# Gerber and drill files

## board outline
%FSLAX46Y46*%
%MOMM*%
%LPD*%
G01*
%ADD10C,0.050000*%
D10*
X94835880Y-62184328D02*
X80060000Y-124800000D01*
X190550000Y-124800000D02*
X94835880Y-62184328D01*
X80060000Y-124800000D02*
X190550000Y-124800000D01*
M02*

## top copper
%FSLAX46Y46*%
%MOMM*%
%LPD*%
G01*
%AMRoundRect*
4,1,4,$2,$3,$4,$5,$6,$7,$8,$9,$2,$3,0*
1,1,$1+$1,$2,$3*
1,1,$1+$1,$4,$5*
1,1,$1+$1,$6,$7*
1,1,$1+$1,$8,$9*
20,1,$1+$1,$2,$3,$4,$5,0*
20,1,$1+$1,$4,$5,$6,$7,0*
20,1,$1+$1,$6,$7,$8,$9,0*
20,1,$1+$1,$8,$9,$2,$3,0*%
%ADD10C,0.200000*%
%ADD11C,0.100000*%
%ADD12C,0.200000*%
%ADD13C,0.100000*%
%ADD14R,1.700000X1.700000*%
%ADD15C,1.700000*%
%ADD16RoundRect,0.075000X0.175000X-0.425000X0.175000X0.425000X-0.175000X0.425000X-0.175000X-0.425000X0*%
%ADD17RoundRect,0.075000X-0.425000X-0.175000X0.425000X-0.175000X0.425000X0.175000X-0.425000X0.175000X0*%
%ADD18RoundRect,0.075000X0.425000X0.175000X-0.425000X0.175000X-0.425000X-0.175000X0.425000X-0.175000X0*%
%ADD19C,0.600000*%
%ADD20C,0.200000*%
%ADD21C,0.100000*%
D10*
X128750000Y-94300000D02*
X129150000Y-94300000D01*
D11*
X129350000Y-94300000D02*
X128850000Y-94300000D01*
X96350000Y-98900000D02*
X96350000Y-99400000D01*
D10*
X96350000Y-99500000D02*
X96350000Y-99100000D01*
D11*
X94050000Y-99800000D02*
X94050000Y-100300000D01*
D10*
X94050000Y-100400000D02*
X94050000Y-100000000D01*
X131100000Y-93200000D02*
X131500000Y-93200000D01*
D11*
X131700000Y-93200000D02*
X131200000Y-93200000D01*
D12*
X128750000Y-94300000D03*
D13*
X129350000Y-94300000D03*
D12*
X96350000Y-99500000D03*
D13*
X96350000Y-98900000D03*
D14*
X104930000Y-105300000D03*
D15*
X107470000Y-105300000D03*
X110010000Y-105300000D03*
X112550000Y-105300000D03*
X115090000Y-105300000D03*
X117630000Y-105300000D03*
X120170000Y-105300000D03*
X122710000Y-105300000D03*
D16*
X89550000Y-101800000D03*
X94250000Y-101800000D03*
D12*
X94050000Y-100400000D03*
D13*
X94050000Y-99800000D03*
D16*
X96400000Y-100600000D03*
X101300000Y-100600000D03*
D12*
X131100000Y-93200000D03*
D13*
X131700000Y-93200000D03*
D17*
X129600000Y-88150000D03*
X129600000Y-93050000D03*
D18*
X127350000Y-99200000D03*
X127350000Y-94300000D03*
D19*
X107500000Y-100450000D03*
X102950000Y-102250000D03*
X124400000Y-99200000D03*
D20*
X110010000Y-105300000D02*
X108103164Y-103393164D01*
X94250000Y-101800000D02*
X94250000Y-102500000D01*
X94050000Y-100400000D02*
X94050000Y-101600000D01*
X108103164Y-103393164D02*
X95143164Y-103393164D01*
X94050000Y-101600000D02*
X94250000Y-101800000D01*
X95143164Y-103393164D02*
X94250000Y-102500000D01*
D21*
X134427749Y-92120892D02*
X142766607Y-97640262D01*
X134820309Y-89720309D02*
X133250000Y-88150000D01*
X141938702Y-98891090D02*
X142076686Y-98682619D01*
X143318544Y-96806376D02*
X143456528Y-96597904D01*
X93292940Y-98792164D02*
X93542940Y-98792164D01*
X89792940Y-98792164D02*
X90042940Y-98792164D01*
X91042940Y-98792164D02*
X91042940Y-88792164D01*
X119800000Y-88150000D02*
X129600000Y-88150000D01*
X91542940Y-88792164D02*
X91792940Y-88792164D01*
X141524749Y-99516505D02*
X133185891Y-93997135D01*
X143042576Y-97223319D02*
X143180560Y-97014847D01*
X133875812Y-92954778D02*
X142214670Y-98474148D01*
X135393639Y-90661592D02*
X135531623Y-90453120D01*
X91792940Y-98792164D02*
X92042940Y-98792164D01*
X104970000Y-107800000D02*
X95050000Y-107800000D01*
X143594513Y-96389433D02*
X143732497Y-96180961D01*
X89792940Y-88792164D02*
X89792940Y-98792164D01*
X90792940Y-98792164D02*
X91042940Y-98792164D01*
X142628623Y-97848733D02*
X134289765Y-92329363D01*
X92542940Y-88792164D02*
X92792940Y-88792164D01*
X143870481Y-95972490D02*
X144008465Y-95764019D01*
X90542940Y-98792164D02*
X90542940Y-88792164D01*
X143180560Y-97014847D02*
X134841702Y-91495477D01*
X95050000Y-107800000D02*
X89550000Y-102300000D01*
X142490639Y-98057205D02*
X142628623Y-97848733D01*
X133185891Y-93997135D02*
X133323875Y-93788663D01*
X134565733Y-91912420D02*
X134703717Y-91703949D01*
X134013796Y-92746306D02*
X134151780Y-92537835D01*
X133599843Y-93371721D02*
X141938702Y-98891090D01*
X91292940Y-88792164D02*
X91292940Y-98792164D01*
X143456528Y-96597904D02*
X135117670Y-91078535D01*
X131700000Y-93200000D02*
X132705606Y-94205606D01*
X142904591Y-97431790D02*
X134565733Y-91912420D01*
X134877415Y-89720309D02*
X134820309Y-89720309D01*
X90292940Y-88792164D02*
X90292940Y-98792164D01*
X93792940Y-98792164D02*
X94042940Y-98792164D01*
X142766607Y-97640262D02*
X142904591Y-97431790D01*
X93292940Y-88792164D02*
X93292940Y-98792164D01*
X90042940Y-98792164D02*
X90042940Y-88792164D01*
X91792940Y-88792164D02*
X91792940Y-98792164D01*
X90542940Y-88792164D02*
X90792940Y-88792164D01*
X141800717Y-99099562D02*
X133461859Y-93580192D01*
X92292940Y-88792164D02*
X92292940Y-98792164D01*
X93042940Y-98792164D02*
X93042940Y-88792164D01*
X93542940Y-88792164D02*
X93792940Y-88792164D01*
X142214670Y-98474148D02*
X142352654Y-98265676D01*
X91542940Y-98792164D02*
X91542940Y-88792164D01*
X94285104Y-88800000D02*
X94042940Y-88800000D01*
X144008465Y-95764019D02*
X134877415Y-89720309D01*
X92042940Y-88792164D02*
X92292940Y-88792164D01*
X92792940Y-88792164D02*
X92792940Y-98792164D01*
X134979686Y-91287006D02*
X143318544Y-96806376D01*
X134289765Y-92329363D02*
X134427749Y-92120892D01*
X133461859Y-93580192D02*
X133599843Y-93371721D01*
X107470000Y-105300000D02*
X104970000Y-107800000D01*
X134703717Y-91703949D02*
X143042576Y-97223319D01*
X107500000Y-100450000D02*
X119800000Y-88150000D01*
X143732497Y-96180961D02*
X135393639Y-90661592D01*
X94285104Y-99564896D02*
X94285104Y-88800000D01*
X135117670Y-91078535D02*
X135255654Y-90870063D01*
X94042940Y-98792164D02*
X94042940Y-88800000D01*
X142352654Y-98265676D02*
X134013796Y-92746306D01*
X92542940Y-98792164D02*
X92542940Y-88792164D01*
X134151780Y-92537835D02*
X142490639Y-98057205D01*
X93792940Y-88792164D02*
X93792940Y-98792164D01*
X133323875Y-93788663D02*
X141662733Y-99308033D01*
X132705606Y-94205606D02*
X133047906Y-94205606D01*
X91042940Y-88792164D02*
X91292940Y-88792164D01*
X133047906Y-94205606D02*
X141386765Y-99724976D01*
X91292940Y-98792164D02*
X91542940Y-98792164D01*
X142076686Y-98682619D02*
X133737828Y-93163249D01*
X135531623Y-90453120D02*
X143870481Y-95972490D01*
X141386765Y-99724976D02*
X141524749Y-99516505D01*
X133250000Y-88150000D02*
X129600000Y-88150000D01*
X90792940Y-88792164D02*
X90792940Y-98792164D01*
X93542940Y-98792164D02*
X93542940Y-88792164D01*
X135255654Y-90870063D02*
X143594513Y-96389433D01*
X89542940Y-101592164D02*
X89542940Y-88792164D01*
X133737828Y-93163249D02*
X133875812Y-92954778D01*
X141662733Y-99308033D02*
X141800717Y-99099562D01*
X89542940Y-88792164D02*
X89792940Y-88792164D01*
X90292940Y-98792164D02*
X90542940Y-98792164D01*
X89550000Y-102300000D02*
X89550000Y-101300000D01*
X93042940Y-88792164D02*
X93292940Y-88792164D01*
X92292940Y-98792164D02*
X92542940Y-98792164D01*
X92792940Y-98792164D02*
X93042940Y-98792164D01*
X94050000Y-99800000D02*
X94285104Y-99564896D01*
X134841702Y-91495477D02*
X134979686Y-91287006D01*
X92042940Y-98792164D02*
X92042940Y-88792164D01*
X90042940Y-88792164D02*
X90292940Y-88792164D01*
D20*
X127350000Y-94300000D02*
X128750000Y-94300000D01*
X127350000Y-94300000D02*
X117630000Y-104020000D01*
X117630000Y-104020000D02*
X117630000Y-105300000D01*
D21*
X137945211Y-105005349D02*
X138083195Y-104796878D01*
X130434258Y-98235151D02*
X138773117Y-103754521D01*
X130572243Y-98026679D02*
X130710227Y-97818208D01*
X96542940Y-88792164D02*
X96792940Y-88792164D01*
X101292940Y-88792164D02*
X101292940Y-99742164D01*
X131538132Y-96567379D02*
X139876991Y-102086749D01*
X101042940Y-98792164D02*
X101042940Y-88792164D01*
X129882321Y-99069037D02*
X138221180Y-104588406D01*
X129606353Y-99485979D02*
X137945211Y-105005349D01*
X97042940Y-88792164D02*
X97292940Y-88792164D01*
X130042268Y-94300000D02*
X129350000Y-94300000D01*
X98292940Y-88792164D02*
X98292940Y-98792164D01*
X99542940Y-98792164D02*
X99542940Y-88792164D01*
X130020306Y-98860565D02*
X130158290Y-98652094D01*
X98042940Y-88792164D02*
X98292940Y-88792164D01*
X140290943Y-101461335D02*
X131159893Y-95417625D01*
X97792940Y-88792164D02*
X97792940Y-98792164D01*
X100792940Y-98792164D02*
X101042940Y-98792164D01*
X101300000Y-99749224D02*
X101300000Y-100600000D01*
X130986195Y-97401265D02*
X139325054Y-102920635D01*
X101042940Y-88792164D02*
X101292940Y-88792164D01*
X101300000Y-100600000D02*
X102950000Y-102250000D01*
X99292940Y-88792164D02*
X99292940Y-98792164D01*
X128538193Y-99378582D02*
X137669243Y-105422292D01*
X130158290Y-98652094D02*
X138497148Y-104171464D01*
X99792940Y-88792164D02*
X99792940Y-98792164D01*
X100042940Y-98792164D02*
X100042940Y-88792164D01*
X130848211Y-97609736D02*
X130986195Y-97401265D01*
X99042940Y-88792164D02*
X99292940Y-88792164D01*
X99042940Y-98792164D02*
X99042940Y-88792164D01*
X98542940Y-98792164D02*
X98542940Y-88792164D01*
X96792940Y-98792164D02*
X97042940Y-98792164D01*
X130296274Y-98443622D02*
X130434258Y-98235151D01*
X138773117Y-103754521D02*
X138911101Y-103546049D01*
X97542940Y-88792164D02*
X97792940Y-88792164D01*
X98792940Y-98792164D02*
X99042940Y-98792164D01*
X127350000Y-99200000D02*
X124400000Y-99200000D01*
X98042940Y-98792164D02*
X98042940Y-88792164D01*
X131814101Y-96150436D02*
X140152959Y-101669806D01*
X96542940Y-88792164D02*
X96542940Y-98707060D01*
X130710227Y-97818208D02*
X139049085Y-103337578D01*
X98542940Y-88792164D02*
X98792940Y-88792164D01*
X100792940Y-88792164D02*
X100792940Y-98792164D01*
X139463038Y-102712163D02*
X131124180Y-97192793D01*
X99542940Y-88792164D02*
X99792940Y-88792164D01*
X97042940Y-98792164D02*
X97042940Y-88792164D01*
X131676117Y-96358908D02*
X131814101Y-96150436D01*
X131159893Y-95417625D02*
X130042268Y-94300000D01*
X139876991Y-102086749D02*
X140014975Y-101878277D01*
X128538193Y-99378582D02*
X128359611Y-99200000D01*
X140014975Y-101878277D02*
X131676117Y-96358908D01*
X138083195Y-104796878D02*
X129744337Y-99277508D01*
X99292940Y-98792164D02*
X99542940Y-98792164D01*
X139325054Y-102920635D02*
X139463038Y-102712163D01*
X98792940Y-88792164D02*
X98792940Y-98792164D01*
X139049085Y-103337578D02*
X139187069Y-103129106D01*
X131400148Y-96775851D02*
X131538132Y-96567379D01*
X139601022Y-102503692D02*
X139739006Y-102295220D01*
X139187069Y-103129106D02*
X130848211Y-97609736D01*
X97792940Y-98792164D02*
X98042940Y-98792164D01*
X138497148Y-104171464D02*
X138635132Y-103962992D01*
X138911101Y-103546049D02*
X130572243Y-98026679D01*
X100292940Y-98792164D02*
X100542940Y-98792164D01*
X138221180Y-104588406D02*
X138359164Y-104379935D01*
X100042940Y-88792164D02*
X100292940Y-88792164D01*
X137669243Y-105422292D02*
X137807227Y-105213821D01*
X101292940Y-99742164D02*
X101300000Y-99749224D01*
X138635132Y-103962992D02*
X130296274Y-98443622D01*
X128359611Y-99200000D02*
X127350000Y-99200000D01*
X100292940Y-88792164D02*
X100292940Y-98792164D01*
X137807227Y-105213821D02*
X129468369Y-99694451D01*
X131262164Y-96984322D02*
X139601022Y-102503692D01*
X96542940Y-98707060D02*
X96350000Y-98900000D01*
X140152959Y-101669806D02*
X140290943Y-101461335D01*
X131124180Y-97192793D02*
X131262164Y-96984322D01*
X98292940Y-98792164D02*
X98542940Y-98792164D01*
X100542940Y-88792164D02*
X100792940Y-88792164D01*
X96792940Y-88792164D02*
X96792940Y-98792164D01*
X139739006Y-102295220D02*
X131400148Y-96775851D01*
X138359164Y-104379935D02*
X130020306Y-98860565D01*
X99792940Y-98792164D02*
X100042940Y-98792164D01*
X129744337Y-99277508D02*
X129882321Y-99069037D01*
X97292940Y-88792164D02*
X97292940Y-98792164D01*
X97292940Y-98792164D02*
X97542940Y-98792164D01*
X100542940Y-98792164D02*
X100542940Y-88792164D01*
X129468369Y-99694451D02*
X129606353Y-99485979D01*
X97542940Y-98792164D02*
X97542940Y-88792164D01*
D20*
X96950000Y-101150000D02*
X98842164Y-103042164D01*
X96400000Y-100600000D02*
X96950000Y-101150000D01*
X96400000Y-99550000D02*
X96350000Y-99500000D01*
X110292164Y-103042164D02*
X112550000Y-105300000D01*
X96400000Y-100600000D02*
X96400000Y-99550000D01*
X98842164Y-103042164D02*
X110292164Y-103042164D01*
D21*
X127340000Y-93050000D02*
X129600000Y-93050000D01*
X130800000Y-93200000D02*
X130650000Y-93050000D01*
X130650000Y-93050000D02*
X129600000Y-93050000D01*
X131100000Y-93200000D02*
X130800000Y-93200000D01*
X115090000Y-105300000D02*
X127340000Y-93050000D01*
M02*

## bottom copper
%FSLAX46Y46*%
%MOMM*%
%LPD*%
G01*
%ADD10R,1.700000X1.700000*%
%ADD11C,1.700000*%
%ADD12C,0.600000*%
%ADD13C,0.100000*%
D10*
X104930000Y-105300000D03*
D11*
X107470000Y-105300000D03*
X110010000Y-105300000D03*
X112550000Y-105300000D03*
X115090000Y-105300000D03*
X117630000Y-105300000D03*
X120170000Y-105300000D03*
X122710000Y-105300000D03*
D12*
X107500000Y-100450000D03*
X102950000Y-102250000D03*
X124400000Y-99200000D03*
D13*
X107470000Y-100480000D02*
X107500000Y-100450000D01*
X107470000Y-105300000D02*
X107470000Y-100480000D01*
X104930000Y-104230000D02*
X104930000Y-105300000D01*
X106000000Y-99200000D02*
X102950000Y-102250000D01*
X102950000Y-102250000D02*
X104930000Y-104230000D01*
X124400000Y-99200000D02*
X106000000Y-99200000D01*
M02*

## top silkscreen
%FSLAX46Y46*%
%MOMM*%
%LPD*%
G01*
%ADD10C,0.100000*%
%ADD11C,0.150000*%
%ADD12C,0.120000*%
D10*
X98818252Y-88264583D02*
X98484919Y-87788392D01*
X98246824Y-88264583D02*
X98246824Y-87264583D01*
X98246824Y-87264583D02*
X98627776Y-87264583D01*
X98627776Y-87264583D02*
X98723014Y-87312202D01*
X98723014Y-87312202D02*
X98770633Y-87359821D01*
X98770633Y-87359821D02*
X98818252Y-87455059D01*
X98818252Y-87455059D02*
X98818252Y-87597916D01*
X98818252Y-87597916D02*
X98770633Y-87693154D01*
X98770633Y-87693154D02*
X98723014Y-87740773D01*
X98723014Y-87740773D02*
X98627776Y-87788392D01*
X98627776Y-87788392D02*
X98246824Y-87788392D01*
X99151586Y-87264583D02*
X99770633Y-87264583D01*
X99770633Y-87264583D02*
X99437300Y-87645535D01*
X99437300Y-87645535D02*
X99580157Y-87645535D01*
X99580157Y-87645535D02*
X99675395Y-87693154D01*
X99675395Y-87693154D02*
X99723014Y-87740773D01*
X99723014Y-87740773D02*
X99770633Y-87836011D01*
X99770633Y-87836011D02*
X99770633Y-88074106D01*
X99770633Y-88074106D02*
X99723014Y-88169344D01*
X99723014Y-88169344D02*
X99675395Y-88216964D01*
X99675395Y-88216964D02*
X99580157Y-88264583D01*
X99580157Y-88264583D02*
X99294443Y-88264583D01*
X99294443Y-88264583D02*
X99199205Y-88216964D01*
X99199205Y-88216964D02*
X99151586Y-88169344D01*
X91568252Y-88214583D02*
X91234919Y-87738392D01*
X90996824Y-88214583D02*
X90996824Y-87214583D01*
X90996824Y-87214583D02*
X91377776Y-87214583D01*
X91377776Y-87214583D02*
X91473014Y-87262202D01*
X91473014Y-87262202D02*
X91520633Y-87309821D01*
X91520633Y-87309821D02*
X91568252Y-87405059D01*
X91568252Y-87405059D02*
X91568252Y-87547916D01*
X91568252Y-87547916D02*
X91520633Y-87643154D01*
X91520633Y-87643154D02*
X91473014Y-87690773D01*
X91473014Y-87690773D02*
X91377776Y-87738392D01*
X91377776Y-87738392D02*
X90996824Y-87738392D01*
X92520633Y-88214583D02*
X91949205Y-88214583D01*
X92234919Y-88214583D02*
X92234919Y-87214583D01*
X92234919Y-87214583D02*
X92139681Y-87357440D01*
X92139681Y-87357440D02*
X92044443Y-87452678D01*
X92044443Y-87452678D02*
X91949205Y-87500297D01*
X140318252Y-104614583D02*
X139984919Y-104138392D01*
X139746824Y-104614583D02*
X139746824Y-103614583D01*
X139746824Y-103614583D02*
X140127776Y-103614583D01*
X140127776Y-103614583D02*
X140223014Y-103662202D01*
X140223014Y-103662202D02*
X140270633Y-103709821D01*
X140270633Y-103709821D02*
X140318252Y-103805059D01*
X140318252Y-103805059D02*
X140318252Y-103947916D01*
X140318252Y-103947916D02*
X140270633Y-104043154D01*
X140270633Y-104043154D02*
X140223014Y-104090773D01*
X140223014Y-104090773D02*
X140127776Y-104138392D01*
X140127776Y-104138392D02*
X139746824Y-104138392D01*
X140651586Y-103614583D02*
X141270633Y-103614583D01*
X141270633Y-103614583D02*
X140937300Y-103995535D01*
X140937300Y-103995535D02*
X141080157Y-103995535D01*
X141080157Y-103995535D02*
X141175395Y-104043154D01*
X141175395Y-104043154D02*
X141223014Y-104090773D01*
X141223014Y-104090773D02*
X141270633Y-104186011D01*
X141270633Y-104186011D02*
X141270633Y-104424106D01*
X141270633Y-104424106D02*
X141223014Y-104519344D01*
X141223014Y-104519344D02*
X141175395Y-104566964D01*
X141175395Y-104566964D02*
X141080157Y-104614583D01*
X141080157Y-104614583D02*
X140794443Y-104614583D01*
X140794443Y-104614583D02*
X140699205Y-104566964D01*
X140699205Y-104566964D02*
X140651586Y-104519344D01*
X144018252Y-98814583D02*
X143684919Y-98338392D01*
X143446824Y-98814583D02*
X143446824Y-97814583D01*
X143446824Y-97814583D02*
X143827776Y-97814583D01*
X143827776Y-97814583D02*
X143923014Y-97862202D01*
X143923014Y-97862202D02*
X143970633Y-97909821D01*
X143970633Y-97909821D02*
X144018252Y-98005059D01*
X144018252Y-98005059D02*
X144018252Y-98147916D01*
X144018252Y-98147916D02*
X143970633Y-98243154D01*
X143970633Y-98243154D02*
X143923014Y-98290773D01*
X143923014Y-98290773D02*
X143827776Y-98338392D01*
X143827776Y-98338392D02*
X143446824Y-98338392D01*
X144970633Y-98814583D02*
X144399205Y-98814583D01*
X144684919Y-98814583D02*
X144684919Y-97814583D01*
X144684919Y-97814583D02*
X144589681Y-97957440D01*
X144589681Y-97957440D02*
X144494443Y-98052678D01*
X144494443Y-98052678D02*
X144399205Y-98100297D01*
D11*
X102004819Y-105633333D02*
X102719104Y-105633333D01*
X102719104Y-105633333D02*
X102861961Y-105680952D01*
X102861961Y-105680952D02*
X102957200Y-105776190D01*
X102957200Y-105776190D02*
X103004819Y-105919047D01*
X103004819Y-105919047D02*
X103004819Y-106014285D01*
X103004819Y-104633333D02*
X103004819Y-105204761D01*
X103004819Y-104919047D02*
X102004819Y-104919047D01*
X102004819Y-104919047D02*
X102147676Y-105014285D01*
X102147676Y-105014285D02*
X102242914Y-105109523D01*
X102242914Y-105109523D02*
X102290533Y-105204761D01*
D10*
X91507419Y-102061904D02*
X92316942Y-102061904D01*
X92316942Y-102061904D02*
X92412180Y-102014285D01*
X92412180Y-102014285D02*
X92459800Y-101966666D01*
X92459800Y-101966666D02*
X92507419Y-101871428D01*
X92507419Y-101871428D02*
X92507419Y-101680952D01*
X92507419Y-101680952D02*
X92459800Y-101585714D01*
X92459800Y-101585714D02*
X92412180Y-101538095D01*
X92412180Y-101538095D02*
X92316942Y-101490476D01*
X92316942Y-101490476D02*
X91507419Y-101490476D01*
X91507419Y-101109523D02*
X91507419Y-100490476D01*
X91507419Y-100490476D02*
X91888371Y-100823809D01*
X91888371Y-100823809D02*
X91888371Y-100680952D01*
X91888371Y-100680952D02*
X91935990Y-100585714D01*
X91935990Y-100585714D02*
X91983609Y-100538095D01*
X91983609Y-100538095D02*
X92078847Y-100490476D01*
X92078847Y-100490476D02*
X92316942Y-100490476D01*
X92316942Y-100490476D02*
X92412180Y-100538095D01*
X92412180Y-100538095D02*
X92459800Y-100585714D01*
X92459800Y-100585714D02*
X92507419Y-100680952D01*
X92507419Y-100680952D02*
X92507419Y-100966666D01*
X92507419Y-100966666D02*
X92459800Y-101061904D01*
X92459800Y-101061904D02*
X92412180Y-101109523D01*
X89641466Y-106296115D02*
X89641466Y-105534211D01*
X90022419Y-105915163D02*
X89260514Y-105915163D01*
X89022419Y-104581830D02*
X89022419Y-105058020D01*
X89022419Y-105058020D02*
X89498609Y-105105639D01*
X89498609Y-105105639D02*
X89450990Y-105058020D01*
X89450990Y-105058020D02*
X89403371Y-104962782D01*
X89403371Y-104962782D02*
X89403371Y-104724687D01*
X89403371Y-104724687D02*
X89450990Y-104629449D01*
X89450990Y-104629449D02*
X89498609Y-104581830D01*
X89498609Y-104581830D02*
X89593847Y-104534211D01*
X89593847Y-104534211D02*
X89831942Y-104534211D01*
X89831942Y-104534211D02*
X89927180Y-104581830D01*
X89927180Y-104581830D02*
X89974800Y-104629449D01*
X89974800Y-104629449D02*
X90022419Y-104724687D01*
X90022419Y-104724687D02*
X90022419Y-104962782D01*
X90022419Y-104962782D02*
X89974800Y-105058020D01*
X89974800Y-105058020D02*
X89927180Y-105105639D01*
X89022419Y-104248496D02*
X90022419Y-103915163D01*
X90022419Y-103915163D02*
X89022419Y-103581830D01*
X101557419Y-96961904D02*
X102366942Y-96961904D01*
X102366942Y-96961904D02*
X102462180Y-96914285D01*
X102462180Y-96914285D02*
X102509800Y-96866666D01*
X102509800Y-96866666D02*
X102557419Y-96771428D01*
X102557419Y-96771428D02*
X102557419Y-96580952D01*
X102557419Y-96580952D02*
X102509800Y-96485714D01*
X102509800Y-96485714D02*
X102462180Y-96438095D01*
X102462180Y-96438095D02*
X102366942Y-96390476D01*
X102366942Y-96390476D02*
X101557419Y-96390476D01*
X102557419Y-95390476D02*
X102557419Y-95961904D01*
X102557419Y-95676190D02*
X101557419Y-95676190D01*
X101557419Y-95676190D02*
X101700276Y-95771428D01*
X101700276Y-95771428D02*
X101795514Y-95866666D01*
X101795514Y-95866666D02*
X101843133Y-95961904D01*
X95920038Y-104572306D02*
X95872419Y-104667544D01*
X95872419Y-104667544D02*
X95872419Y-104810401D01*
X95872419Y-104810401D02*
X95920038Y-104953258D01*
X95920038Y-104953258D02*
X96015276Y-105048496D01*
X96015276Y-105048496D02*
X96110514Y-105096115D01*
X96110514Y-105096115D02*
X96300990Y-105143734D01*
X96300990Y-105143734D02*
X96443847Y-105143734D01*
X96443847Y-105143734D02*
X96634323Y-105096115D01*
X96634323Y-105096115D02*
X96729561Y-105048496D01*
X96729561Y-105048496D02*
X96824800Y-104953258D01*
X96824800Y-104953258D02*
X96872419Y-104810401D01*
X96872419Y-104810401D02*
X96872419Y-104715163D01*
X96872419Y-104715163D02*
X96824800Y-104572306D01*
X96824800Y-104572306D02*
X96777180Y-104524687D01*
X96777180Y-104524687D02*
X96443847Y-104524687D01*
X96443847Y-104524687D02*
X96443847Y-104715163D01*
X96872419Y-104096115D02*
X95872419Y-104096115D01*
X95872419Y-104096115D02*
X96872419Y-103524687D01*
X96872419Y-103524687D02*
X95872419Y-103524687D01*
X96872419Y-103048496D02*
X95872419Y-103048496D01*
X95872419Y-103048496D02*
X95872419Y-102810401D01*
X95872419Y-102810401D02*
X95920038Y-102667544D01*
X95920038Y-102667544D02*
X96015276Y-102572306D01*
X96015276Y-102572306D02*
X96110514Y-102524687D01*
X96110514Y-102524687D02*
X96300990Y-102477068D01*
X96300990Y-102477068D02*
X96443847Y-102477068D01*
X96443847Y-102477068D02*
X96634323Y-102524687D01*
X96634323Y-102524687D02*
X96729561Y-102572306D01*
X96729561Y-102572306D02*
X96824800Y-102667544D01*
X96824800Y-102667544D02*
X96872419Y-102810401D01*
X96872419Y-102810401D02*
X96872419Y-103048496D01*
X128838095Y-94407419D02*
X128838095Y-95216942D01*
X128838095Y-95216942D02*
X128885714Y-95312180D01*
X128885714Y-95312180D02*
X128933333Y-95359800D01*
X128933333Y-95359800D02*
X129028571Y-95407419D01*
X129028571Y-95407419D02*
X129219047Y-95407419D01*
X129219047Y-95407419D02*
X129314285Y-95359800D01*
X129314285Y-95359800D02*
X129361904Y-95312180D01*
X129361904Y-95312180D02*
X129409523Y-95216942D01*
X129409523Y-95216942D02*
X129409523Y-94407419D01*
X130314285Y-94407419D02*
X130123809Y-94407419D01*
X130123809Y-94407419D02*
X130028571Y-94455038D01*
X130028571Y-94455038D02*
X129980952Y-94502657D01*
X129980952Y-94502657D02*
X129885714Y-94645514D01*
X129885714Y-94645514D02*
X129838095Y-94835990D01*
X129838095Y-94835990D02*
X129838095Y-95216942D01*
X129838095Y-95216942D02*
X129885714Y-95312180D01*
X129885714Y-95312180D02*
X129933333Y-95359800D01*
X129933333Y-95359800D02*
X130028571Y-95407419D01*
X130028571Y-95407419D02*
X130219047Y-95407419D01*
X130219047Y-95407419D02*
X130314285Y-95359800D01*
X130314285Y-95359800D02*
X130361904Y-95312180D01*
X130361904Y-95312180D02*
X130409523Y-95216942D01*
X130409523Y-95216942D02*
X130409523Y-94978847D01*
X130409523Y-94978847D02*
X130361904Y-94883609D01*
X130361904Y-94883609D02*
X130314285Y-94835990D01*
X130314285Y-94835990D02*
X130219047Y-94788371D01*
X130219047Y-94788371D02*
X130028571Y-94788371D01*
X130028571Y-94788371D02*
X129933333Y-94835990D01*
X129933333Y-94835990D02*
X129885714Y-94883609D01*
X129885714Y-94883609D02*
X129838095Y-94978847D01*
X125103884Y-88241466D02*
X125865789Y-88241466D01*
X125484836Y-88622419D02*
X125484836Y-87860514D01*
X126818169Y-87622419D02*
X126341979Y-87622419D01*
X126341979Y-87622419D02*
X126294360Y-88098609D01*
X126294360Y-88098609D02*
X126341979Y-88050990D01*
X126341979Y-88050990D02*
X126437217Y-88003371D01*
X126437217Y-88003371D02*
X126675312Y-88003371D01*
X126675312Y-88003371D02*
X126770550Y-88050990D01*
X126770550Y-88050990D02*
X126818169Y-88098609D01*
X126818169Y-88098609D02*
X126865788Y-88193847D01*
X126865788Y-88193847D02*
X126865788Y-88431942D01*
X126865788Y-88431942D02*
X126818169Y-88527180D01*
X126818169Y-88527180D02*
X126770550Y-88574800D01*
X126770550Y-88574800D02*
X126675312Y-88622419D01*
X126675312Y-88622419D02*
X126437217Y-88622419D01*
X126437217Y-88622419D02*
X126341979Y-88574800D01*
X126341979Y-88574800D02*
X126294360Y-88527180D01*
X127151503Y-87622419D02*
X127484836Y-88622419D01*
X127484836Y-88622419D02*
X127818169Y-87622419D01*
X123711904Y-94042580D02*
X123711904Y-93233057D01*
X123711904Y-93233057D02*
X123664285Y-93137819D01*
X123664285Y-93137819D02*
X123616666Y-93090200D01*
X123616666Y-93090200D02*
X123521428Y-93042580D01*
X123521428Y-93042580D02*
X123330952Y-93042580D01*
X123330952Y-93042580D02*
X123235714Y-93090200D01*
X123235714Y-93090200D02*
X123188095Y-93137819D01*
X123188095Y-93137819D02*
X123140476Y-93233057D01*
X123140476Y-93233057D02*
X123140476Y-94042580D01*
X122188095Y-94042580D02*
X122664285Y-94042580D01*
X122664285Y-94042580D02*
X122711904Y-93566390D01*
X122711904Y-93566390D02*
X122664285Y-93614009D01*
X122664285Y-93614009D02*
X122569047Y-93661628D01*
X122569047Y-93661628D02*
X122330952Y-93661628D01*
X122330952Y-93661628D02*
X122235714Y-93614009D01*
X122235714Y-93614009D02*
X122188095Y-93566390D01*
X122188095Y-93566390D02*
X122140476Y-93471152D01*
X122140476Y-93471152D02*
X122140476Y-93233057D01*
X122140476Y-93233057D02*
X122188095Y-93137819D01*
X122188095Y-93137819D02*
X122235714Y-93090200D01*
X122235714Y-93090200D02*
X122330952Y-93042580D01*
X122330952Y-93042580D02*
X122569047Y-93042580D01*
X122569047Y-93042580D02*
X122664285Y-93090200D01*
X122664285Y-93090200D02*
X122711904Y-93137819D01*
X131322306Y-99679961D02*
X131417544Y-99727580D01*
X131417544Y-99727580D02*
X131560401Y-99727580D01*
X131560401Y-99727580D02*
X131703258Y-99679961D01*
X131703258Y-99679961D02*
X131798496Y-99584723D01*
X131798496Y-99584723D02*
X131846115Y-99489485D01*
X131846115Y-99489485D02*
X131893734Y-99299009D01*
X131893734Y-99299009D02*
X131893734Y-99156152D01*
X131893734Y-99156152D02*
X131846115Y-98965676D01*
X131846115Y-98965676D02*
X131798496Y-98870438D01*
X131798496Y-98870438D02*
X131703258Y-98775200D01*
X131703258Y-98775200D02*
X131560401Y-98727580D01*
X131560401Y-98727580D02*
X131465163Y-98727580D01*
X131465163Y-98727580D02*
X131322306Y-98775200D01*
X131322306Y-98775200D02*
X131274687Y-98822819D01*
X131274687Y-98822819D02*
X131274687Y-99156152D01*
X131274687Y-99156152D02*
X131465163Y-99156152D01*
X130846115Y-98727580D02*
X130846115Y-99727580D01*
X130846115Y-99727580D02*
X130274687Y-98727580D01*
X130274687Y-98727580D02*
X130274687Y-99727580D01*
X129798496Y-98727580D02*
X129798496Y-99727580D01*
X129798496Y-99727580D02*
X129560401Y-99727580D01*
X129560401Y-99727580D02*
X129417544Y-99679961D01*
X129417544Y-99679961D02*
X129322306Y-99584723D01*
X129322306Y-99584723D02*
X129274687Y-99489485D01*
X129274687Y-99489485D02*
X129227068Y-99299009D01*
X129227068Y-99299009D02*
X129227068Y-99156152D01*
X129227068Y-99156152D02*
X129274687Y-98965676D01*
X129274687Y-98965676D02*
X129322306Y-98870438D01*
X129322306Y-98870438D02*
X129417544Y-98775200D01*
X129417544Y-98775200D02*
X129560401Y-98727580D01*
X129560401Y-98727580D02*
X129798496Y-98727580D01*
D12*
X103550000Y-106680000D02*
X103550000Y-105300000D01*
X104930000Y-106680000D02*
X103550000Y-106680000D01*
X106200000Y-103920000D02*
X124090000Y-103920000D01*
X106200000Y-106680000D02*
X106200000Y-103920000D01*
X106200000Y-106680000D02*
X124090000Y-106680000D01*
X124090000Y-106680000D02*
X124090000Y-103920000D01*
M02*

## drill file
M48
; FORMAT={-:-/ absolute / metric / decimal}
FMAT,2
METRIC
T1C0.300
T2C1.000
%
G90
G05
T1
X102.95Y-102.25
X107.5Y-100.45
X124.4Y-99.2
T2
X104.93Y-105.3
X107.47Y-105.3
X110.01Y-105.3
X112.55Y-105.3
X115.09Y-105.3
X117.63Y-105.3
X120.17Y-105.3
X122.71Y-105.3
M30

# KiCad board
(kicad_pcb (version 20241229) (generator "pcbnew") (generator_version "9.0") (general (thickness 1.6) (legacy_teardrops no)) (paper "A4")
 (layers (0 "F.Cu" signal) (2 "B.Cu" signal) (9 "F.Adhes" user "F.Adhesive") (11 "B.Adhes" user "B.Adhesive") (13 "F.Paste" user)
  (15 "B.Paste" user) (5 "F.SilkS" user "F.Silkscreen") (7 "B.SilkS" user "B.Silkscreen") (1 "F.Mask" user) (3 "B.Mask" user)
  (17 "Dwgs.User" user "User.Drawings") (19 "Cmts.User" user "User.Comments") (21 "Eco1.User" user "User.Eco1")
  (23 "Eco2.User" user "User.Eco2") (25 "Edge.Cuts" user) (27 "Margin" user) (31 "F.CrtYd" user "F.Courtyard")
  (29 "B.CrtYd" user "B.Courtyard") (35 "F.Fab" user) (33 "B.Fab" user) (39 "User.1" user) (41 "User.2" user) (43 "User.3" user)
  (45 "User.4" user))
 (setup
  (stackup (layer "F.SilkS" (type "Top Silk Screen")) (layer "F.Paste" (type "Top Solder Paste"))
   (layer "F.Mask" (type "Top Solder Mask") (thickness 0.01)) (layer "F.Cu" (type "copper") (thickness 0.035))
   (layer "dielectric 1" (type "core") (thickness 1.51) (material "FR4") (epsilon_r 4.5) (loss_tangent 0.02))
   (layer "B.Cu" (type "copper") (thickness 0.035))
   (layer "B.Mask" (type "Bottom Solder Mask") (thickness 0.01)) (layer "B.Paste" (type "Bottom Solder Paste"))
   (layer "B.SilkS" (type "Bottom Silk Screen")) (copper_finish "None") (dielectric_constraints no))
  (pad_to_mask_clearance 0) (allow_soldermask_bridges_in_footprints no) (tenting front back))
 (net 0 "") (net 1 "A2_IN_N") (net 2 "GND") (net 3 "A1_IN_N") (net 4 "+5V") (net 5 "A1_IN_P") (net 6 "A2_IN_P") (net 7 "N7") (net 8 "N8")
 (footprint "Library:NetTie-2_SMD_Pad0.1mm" (layer "F.Cu") (at 128.85 94.3)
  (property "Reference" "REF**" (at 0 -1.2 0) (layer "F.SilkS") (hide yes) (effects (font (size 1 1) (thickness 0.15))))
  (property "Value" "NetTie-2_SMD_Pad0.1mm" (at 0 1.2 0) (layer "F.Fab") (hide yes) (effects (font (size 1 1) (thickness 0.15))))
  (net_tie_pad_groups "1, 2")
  (fp_line (start -0.1 0) (end 0.3 0) (stroke (width 0.2) (type solid)) (layer "F.Cu"))
  (fp_line (start 0.5 0) (end 0 0) (stroke (width 0.1) (type solid)) (layer "F.Cu"))
  (pad "1" smd circle (at -0.1 0) (size 0.2 0.2) (layers "F.Cu") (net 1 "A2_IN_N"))
  (pad "2" smd circle (at 0.5 0) (size 0.1 0.1) (layers "F.Cu") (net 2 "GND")))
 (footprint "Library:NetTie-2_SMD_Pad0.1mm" (layer "F.Cu") (at 96.35 99.4 90)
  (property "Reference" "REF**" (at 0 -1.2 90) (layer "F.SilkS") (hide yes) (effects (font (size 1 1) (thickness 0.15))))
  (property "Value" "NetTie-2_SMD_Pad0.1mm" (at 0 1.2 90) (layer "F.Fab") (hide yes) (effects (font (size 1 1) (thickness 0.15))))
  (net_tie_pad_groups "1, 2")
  (fp_line (start 0.5 0) (end 0 0) (stroke (width 0.1) (type solid)) (layer "F.Cu"))
  (fp_line (start -0.1 0) (end 0.3 0) (stroke (width 0.2) (type solid)) (layer "F.Cu"))
  (pad "1" smd circle (at -0.1 0 90) (size 0.2 0.2) (layers "F.Cu") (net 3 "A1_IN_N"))
  (pad "2" smd circle (at 0.5 0 90) (size 0.1 0.1) (layers "F.Cu") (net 2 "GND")))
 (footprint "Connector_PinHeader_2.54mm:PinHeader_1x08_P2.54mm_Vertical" (layer "F.Cu") (at 104.93 105.3 90)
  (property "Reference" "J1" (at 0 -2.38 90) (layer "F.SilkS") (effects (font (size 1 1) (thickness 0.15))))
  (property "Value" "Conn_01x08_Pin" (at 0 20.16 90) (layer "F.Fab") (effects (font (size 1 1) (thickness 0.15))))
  (fp_line (start -1.38 -1.38) (end 0 -1.38) (stroke (width 0.12) (type solid)) (layer "F.SilkS"))
  (fp_line (start -1.38 0) (end -1.38 -1.38) (stroke (width 0.12) (type solid)) (layer "F.SilkS"))
  (fp_line (start 1.38 1.27) (end 1.38 19.16) (stroke (width 0.12) (type solid)) (layer "F.SilkS"))
  (fp_line (start -1.38 1.27) (end 1.38 1.27) (stroke (width 0.12) (type solid)) (layer "F.SilkS"))
  (fp_line (start -1.38 1.27) (end -1.38 19.16) (stroke (width 0.12) (type solid)) (layer "F.SilkS"))
  (fp_line (start -1.38 19.16) (end 1.38 19.16) (stroke (width 0.12) (type solid)) (layer "F.SilkS"))
  (pad "1" thru_hole rect (at 0 0 90) (size 1.7 1.7) (drill 1) (layers "*.Cu" "*.Mask") (remove_unused_layers no) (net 2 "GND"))
  (pad "2" thru_hole circle (at 0 2.54 90) (size 1.7 1.7) (drill 1) (layers "*.Cu" "*.Mask") (remove_unused_layers no) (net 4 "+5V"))
  (pad "3" thru_hole circle (at 0 5.08 90) (size 1.7 1.7) (drill 1) (layers "*.Cu" "*.Mask") (remove_unused_layers no) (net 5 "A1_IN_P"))
  (pad "4" thru_hole circle (at 0 7.62 90) (size 1.7 1.7) (drill 1) (layers "*.Cu" "*.Mask") (remove_unused_layers no) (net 3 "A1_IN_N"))
  (pad "5" thru_hole circle (at 0 10.16 90) (size 1.7 1.7) (drill 1) (layers "*.Cu" "*.Mask") (remove_unused_layers no) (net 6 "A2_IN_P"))
  (pad "6" thru_hole circle (at 0 12.7 90) (size 1.7 1.7) (drill 1) (layers "*.Cu" "*.Mask") (remove_unused_layers no) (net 1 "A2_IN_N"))
  (pad "7" thru_hole circle (at 0 15.24 90) (size 1.7 1.7) (drill 1) (layers "*.Cu" "*.Mask") (remove_unused_layers no) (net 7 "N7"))
  (pad "8" thru_hole circle (at 0 17.78 90) (size 1.7 1.7) (drill 1) (layers "*.Cu" "*.Mask") (remove_unused_layers no) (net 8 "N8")))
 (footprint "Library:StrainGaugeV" (layer "F.Cu") (at 96.85 101.8 90)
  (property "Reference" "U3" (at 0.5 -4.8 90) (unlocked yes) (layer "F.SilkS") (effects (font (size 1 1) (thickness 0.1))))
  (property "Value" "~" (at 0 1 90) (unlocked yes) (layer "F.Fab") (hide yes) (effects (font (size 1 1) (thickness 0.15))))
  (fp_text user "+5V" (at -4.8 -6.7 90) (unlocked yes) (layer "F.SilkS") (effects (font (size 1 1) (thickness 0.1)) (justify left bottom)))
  (pad "1" smd roundrect (at 0 -7.3 90) (size 1 0.5) (layers "F.Cu" "F.Mask" "F.Paste") (roundrect_rratio 0.15) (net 4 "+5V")
   (thermal_bridge_angle 45))
  (pad "2" smd roundrect (at 0 -2.6 90) (size 1 0.5) (layers "F.Cu" "F.Mask" "F.Paste") (roundrect_rratio 0.15) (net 5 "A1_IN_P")
   (thermal_bridge_angle 45)))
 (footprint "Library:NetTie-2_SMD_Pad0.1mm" (layer "F.Cu") (at 94.05 100.3 90)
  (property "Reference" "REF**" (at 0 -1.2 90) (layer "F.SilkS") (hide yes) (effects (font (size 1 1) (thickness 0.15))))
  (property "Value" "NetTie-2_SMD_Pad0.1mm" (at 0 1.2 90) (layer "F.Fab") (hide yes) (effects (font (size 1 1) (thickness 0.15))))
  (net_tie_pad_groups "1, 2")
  (fp_line (start 0.5 0) (end 0 0) (stroke (width 0.1) (type solid)) (layer "F.Cu"))
  (fp_line (start -0.1 0) (end 0.3 0) (stroke (width 0.2) (type solid)) (layer "F.Cu"))
  (pad "1" smd circle (at -0.1 0 90) (size 0.2 0.2) (layers "F.Cu") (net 5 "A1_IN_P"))
  (pad "2" smd circle (at 0.5 0 90) (size 0.1 0.1) (layers "F.Cu") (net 4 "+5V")))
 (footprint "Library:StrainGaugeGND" (layer "F.Cu") (at 101.3 100.6 90)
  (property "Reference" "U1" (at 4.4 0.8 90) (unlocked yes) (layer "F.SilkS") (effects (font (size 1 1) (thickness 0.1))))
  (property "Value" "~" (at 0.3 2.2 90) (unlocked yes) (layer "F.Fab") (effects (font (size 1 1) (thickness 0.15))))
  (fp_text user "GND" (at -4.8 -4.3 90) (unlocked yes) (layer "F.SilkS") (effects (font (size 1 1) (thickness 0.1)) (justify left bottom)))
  (pad "1" smd roundrect (at 0 -4.9 90) (size 1 0.5) (layers "F.Cu" "F.Mask" "F.Paste") (roundrect_rratio 0.15) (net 3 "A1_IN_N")
   (thermal_bridge_angle 45))
  (pad "2" smd roundrect (at 0 0 90) (size 1 0.5) (layers "F.Cu" "F.Mask" "F.Paste") (roundrect_rratio 0.15) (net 2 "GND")
   (thermal_bridge_angle 45)))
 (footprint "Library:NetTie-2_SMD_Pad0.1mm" (layer "F.Cu") (at 131.2 93.2)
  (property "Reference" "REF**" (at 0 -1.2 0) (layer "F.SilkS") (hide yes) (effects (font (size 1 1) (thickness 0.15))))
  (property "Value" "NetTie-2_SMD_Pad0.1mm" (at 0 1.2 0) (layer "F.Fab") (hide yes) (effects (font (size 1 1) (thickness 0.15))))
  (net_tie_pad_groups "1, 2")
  (fp_line (start -0.1 0) (end 0.3 0) (stroke (width 0.2) (type solid)) (layer "F.Cu"))
  (fp_line (start 0.5 0) (end 0 0) (stroke (width 0.1) (type solid)) (layer "F.Cu"))
  (pad "1" smd circle (at -0.1 0) (size 0.2 0.2) (layers "F.Cu") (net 6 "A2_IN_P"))
  (pad "2" smd circle (at 0.5 0) (size 0.1 0.1) (layers "F.Cu") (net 4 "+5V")))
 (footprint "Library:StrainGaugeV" (layer "F.Cu") (at 129.6 95.45)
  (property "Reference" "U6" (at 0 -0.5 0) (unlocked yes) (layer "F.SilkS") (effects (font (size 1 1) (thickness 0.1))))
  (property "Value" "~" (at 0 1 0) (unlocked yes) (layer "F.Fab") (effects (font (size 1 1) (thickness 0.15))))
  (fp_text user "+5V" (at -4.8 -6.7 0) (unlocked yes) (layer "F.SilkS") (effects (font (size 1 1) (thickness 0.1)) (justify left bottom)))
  (pad "1" smd roundrect (at 0 -7.3) (size 1 0.5) (layers "F.Cu" "F.Mask" "F.Paste") (roundrect_rratio 0.15) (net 4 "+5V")
   (thermal_bridge_angle 45))
  (pad "2" smd roundrect (at 0 -2.4) (size 1 0.5) (layers "F.Cu" "F.Mask" "F.Paste") (roundrect_rratio 0.15) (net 6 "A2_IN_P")
   (thermal_bridge_angle 45)))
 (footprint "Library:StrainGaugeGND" (layer "F.Cu") (at 127.35 94.3 180)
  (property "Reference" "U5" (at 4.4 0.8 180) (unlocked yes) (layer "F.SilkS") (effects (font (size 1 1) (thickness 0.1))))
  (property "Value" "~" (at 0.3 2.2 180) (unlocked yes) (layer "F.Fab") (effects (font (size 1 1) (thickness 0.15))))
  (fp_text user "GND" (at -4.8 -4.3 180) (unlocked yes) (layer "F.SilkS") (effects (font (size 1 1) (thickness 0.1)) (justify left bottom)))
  (pad "1" smd roundrect (at 0 -4.9 180) (size 1 0.5) (layers "F.Cu" "F.Mask" "F.Paste") (roundrect_rratio 0.15) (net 2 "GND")
   (thermal_bridge_angle 45))
  (pad "2" smd roundrect (at 0 0 180) (size 1 0.5) (layers "F.Cu" "F.Mask" "F.Paste") (roundrect_rratio 0.15) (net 1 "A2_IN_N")
   (thermal_bridge_angle 45)))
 (gr_line (start 94.83588 62.184328) (end 80.06 124.8) (stroke (width 0.05) (type solid)) (layer "Edge.Cuts"))
 (gr_line (start 190.55 124.8) (end 94.83588 62.184328) (stroke (width 0.05) (type solid)) (layer "Edge.Cuts"))
 (gr_line (start 80.06 124.8) (end 190.55 124.8) (stroke (width 0.05) (type default)) (layer "Edge.Cuts"))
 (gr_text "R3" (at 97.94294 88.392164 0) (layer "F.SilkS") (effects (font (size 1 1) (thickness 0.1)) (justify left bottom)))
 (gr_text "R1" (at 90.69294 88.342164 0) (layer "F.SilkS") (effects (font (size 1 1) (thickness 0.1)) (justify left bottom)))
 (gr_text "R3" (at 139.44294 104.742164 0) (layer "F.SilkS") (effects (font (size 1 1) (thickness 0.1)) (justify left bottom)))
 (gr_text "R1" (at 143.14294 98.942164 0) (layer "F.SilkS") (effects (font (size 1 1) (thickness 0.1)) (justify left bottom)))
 (segment (start 110.01 105.3) (end 108.103164 103.393164) (width 0.2) (layer "F.Cu") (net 5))
 (segment (start 94.25 101.8) (end 94.25 102.5) (width 0.2) (layer "F.Cu") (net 5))
 (segment (start 94.05 100.4) (end 94.05 101.6) (width 0.2) (layer "F.Cu") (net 5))
 (segment (start 108.103164 103.393164) (end 95.143164 103.393164) (width 0.2) (layer "F.Cu") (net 5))
 (segment (start 94.05 101.6) (end 94.25 101.8) (width 0.2) (layer "F.Cu") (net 5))
 (segment (start 95.143164 103.393164) (end 94.25 102.5) (width 0.2) (layer "F.Cu") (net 5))
 (segment (start 134.427749 92.120892) (end 142.766607 97.640262) (width 0.1) (layer "F.Cu") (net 4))
 (segment (start 134.820309 89.720309) (end 133.25 88.15) (width 0.1) (layer "F.Cu") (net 4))
 (segment (start 141.938702 98.89109) (end 142.076686 98.682619) (width 0.1) (layer "F.Cu") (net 4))
 (segment (start 143.318544 96.806376) (end 143.456528 96.597904) (width 0.1) (layer "F.Cu") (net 4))
 (segment (start 93.29294 98.792164) (end 93.54294 98.792164) (width 0.1) (layer "F.Cu") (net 4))
 (segment (start 89.79294 98.792164) (end 90.04294 98.792164) (width 0.1) (layer "F.Cu") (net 4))
 (segment (start 91.04294 98.792164) (end 91.04294 88.792164) (width 0.1) (layer "F.Cu") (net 4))
 (segment (start 119.8 88.15) (end 129.6 88.15) (width 0.1) (layer "F.Cu") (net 4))
 (segment (start 91.54294 88.792164) (end 91.79294 88.792164) (width 0.1) (layer "F.Cu") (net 4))
 (segment (start 141.524749 99.516505) (end 133.185891 93.997135) (width 0.1) (layer "F.Cu") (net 4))
 (segment (start 143.042576 97.223319) (end 143.18056 97.014847) (width 0.1) (layer "F.Cu") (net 4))
 (segment (start 133.875812 92.954778) (end 142.21467 98.474148) (width 0.1) (layer "F.Cu") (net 4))
 (segment (start 135.393639 90.661592) (end 135.531623 90.45312) (width 0.1) (layer "F.Cu") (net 4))
 (segment (start 91.79294 98.792164) (end 92.04294 98.792164) (width 0.1) (layer "F.Cu") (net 4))
 (segment (start 104.97 107.8) (end 95.05 107.8) (width 0.1) (layer "F.Cu") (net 4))
 (segment (start 143.594513 96.389433) (end 143.732497 96.180961) (width 0.1) (layer "F.Cu") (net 4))
 (segment (start 89.79294 88.792164) (end 89.79294 98.792164) (width 0.1) (layer "F.Cu") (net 4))
 (segment (start 90.79294 98.792164) (end 91.04294 98.792164) (width 0.1) (layer "F.Cu") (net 4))
 (segment (start 142.628623 97.848733) (end 134.289765 92.329363) (width 0.1) (layer "F.Cu") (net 4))
 (segment (start 92.54294 88.792164) (end 92.79294 88.792164) (width 0.1) (layer "F.Cu") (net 4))
 (segment (start 143.870481 95.97249) (end 144.008465 95.764019) (width 0.1) (layer "F.Cu") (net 4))
 (segment (start 90.54294 98.792164) (end 90.54294 88.792164) (width 0.1) (layer "F.Cu") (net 4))
 (segment (start 143.18056 97.014847) (end 134.841702 91.495477) (width 0.1) (layer "F.Cu") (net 4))
 (segment (start 95.05 107.8) (end 89.55 102.3) (width 0.1) (layer "F.Cu") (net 4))
 (segment (start 142.490639 98.057205) (end 142.628623 97.848733) (width 0.1) (layer "F.Cu") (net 4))
 (segment (start 133.185891 93.997135) (end 133.323875 93.788663) (width 0.1) (layer "F.Cu") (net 4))
 (segment (start 134.565733 91.91242) (end 134.703717 91.703949) (width 0.1) (layer "F.Cu") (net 4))
 (segment (start 134.013796 92.746306) (end 134.15178 92.537835) (width 0.1) (layer "F.Cu") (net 4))
 (segment (start 133.599843 93.371721) (end 141.938702 98.89109) (width 0.1) (layer "F.Cu") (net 4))
 (segment (start 91.29294 88.792164) (end 91.29294 98.792164) (width 0.1) (layer "F.Cu") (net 4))
 (segment (start 143.456528 96.597904) (end 135.11767 91.078535) (width 0.1) (layer "F.Cu") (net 4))
 (segment (start 131.7 93.2) (end 132.705606 94.205606) (width 0.1) (layer "F.Cu") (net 4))
 (segment (start 142.904591 97.43179) (end 134.565733 91.91242) (width 0.1) (layer "F.Cu") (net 4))
 (segment (start 134.877415 89.720309) (end 134.820309 89.720309) (width 0.1) (layer "F.Cu") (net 4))
 (segment (start 90.29294 88.792164) (end 90.29294 98.792164) (width 0.1) (layer "F.Cu") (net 4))
 (segment (start 93.79294 98.792164) (end 94.04294 98.792164) (width 0.1) (layer "F.Cu") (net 4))
 (segment (start 142.766607 97.640262) (end 142.904591 97.43179) (width 0.1) (layer "F.Cu") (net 4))
 (segment (start 93.29294 88.792164) (end 93.29294 98.792164) (width 0.1) (layer "F.Cu") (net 4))
 (segment (start 90.04294 98.792164) (end 90.04294 88.792164) (width 0.1) (layer "F.Cu") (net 4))
 (segment (start 91.79294 88.792164) (end 91.79294 98.792164) (width 0.1) (layer "F.Cu") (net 4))
 (segment (start 90.54294 88.792164) (end 90.79294 88.792164) (width 0.1) (layer "F.Cu") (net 4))
 (segment (start 141.800717 99.099562) (end 133.461859 93.580192) (width 0.1) (layer "F.Cu") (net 4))
 (segment (start 92.29294 88.792164) (end 92.29294 98.792164) (width 0.1) (layer "F.Cu") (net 4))
 (segment (start 93.04294 98.792164) (end 93.04294 88.792164) (width 0.1) (layer "F.Cu") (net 4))
 (segment (start 93.54294 88.792164) (end 93.79294 88.792164) (width 0.1) (layer "F.Cu") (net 4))
 (segment (start 142.21467 98.474148) (end 142.352654 98.265676) (width 0.1) (layer "F.Cu") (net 4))
 (segment (start 91.54294 98.792164) (end 91.54294 88.792164) (width 0.1) (layer "F.Cu") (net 4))
 (segment (start 94.285104 88.8) (end 94.04294 88.8) (width 0.1) (layer "F.Cu") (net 4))
 (segment (start 144.008465 95.764019) (end 134.877415 89.720309) (width 0.1) (layer "F.Cu") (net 4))
 (segment (start 92.04294 88.792164) (end 92.29294 88.792164) (width 0.1) (layer "F.Cu") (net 4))
 (segment (start 92.79294 88.792164) (end 92.79294 98.792164) (width 0.1) (layer "F.Cu") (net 4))
 (segment (start 134.979686 91.287006) (end 143.318544 96.806376) (width 0.1) (layer "F.Cu") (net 4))
 (segment (start 134.289765 92.329363) (end 134.427749 92.120892) (width 0.1) (layer "F.Cu") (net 4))
 (segment (start 133.461859 93.580192) (end 133.599843 93.371721) (width 0.1) (layer "F.Cu") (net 4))
 (segment (start 107.47 105.3) (end 104.97 107.8) (width 0.1) (layer "F.Cu") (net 4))
 (segment (start 134.703717 91.703949) (end 143.042576 97.223319) (width 0.1) (layer "F.Cu") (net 4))
 (segment (start 107.5 100.45) (end 119.8 88.15) (width 0.1) (layer "F.Cu") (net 4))
 (segment (start 143.732497 96.180961) (end 135.393639 90.661592) (width 0.1) (layer "F.Cu") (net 4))
 (segment (start 94.285104 99.564896) (end 94.285104 88.8) (width 0.1) (layer "F.Cu") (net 4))
 (segment (start 135.11767 91.078535) (end 135.255654 90.870063) (width 0.1) (layer "F.Cu") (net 4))
 (segment (start 94.04294 98.792164) (end 94.04294 88.8) (width 0.1) (layer "F.Cu") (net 4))
 (segment (start 142.352654 98.265676) (end 134.013796 92.746306) (width 0.1) (layer "F.Cu") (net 4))
 (segment (start 92.54294 98.792164) (end 92.54294 88.792164) (width 0.1) (layer "F.Cu") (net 4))
 (segment (start 134.15178 92.537835) (end 142.490639 98.057205) (width 0.1) (layer "F.Cu") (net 4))
 (segment (start 93.79294 88.792164) (end 93.79294 98.792164) (width 0.1) (layer "F.Cu") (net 4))
 (segment (start 133.323875 93.788663) (end 141.662733 99.308033) (width 0.1) (layer "F.Cu") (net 4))
 (segment (start 132.705606 94.205606) (end 133.047906 94.205606) (width 0.1) (layer "F.Cu") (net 4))
 (segment (start 91.04294 88.792164) (end 91.29294 88.792164) (width 0.1) (layer "F.Cu") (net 4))
 (segment (start 133.047906 94.205606) (end 141.386765 99.724976) (width 0.1) (layer "F.Cu") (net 4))
 (segment (start 91.29294 98.792164) (end 91.54294 98.792164) (width 0.1) (layer "F.Cu") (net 4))
 (segment (start 142.076686 98.682619) (end 133.737828 93.163249) (width 0.1) (layer "F.Cu") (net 4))
 (segment (start 135.531623 90.45312) (end 143.870481 95.97249) (width 0.1) (layer "F.Cu") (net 4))
 (segment (start 141.386765 99.724976) (end 141.524749 99.516505) (width 0.1) (layer "F.Cu") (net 4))
 (segment (start 133.25 88.15) (end 129.6 88.15) (width 0.1) (layer "F.Cu") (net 4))
 (segment (start 90.79294 88.792164) (end 90.79294 98.792164) (width 0.1) (layer "F.Cu") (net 4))
 (segment (start 93.54294 98.792164) (end 93.54294 88.792164) (width 0.1) (layer "F.Cu") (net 4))
 (segment (start 135.255654 90.870063) (end 143.594513 96.389433) (width 0.1) (layer "F.Cu") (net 4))
 (segment (start 89.54294 101.592164) (end 89.54294 88.792164) (width 0.1) (layer "F.Cu") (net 4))
 (segment (start 133.737828 93.163249) (end 133.875812 92.954778) (width 0.1) (layer "F.Cu") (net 4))
 (segment (start 141.662733 99.308033) (end 141.800717 99.099562) (width 0.1) (layer "F.Cu") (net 4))
 (segment (start 89.54294 88.792164) (end 89.79294 88.792164) (width 0.1) (layer "F.Cu") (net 4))
 (segment (start 90.29294 98.792164) (end 90.54294 98.792164) (width 0.1) (layer "F.Cu") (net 4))
 (segment (start 89.55 102.3) (end 89.55 101.3) (width 0.1) (layer "F.Cu") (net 4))
 (segment (start 93.04294 88.792164) (end 93.29294 88.792164) (width 0.1) (layer "F.Cu") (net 4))
 (segment (start 92.29294 98.792164) (end 92.54294 98.792164) (width 0.1) (layer "F.Cu") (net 4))
 (segment (start 92.79294 98.792164) (end 93.04294 98.792164) (width 0.1) (layer "F.Cu") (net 4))
 (segment (start 94.05 99.8) (end 94.285104 99.564896) (width 0.1) (layer "F.Cu") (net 4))
 (segment (start 134.841702 91.495477) (end 134.979686 91.287006) (width 0.1) (layer "F.Cu") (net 4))
 (segment (start 92.04294 98.792164) (end 92.04294 88.792164) (width 0.1) (layer "F.Cu") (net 4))
 (segment (start 90.04294 88.792164) (end 90.29294 88.792164) (width 0.1) (layer "F.Cu") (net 4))
 (via (at 107.5 100.45) (size 0.6) (drill 0.3) (layers "F.Cu" "B.Cu") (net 4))
 (segment (start 107.47 100.48) (end 107.5 100.45) (width 0.1) (layer "B.Cu") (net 4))
 (segment (start 107.47 105.3) (end 107.47 100.48) (width 0.1) (layer "B.Cu") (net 4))
 (segment (start 127.35 94.3) (end 128.75 94.3) (width 0.2) (layer "F.Cu") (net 1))
 (segment (start 127.35 94.3) (end 117.63 104.02) (width 0.2) (layer "F.Cu") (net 1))
 (segment (start 117.63 104.02) (end 117.63 105.3) (width 0.2) (layer "F.Cu") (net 1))
 (segment (start 137.945211 105.005349) (end 138.083195 104.796878) (width 0.1) (layer "F.Cu") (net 2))
 (segment (start 130.434258 98.235151) (end 138.773117 103.754521) (width 0.1) (layer "F.Cu") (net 2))
 (segment (start 130.572243 98.026679) (end 130.710227 97.818208) (width 0.1) (layer "F.Cu") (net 2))
 (segment (start 96.54294 88.792164) (end 96.79294 88.792164) (width 0.1) (layer "F.Cu") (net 2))
 (segment (start 101.29294 88.792164) (end 101.29294 99.742164) (width 0.1) (layer "F.Cu") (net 2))
 (segment (start 131.538132 96.567379) (end 139.876991 102.086749) (width 0.1) (layer "F.Cu") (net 2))
 (segment (start 101.04294 98.792164) (end 101.04294 88.792164) (width 0.1) (layer "F.Cu") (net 2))
 (segment (start 129.882321 99.069037) (end 138.22118 104.588406) (width 0.1) (layer "F.Cu") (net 2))
 (segment (start 129.606353 99.485979) (end 137.945211 105.005349) (width 0.1) (layer "F.Cu") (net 2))
 (segment (start 97.04294 88.792164) (end 97.29294 88.792164) (width 0.1) (layer "F.Cu") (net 2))
 (segment (start 130.042268 94.3) (end 129.35 94.3) (width 0.1) (layer "F.Cu") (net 2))
 (segment (start 98.29294 88.792164) (end 98.29294 98.792164) (width 0.1) (layer "F.Cu") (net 2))
 (segment (start 99.54294 98.792164) (end 99.54294 88.792164) (width 0.1) (layer "F.Cu") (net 2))
 (segment (start 130.020306 98.860565) (end 130.15829 98.652094) (width 0.1) (layer "F.Cu") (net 2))
 (segment (start 98.04294 88.792164) (end 98.29294 88.792164) (width 0.1) (layer "F.Cu") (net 2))
 (segment (start 140.290943 101.461335) (end 131.159893 95.417625) (width 0.1) (layer "F.Cu") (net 2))
 (segment (start 97.79294 88.792164) (end 97.79294 98.792164) (width 0.1) (layer "F.Cu") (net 2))
 (segment (start 100.79294 98.792164) (end 101.04294 98.792164) (width 0.1) (layer "F.Cu") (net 2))
 (segment (start 101.3 99.749224) (end 101.3 100.6) (width 0.1) (layer "F.Cu") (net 2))
 (segment (start 130.986195 97.401265) (end 139.325054 102.920635) (width 0.1) (layer "F.Cu") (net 2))
 (segment (start 101.04294 88.792164) (end 101.29294 88.792164) (width 0.1) (layer "F.Cu") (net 2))
 (segment (start 101.3 100.6) (end 102.95 102.25) (width 0.1) (layer "F.Cu") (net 2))
 (segment (start 99.29294 88.792164) (end 99.29294 98.792164) (width 0.1) (layer "F.Cu") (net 2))
 (segment (start 128.538193 99.378582) (end 137.669243 105.422292) (width 0.1) (layer "F.Cu") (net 2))
 (segment (start 130.15829 98.652094) (end 138.497148 104.171464) (width 0.1) (layer "F.Cu") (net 2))
 (segment (start 99.79294 88.792164) (end 99.79294 98.792164) (width 0.1) (layer "F.Cu") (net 2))
 (segment (start 100.04294 98.792164) (end 100.04294 88.792164) (width 0.1) (layer "F.Cu") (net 2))
 (segment (start 130.848211 97.609736) (end 130.986195 97.401265) (width 0.1) (layer "F.Cu") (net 2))
 (segment (start 99.04294 88.792164) (end 99.29294 88.792164) (width 0.1) (layer "F.Cu") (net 2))
 (segment (start 99.04294 98.792164) (end 99.04294 88.792164) (width 0.1) (layer "F.Cu") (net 2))
 (segment (start 98.54294 98.792164) (end 98.54294 88.792164) (width 0.1) (layer "F.Cu") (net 2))
 (segment (start 96.79294 98.792164) (end 97.04294 98.792164) (width 0.1) (layer "F.Cu") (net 2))
 (segment (start 130.296274 98.443622) (end 130.434258 98.235151) (width 0.1) (layer "F.Cu") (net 2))
 (segment (start 138.773117 103.754521) (end 138.911101 103.546049) (width 0.1) (layer "F.Cu") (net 2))
 (segment (start 97.54294 88.792164) (end 97.79294 88.792164) (width 0.1) (layer "F.Cu") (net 2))
 (segment (start 98.79294 98.792164) (end 99.04294 98.792164) (width 0.1) (layer "F.Cu") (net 2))
 (segment (start 127.35 99.2) (end 124.4 99.2) (width 0.1) (layer "F.Cu") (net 2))
 (segment (start 98.04294 98.792164) (end 98.04294 88.792164) (width 0.1) (layer "F.Cu") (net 2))
 (segment (start 131.814101 96.150436) (end 140.152959 101.669806) (width 0.1) (layer "F.Cu") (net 2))
 (segment (start 96.54294 88.792164) (end 96.54294 98.70706) (width 0.1) (layer "F.Cu") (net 2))
 (segment (start 130.710227 97.818208) (end 139.049085 103.337578) (width 0.1) (layer "F.Cu") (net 2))
 (segment (start 98.54294 88.792164) (end 98.79294 88.792164) (width 0.1) (layer "F.Cu") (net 2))
 (segment (start 100.79294 88.792164) (end 100.79294 98.792164) (width 0.1) (layer "F.Cu") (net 2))
 (segment (start 139.463038 102.712163) (end 131.12418 97.192793) (width 0.1) (layer "F.Cu") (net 2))
 (segment (start 99.54294 88.792164) (end 99.79294 88.792164) (width 0.1) (layer "F.Cu") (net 2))
 (segment (start 97.04294 98.792164) (end 97.04294 88.792164) (width 0.1) (layer "F.Cu") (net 2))
 (segment (start 131.676117 96.358908) (end 131.814101 96.150436) (width 0.1) (layer "F.Cu") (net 2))
 (segment (start 131.159893 95.417625) (end 130.042268 94.3) (width 0.1) (layer "F.Cu") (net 2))
 (segment (start 139.876991 102.086749) (end 140.014975 101.878277) (width 0.1) (layer "F.Cu") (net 2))
 (segment (start 128.538193 99.378582) (end 128.359611 99.2) (width 0.1) (layer "F.Cu") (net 2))
 (segment (start 140.014975 101.878277) (end 131.676117 96.358908) (width 0.1) (layer "F.Cu") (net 2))
 (segment (start 138.083195 104.796878) (end 129.744337 99.277508) (width 0.1) (layer "F.Cu") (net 2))
 (segment (start 99.29294 98.792164) (end 99.54294 98.792164) (width 0.1) (layer "F.Cu") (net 2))
 (segment (start 139.325054 102.920635) (end 139.463038 102.712163) (width 0.1) (layer "F.Cu") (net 2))
 (segment (start 98.79294 88.792164) (end 98.79294 98.792164) (width 0.1) (layer "F.Cu") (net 2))
 (segment (start 139.049085 103.337578) (end 139.187069 103.129106) (width 0.1) (layer "F.Cu") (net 2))
 (segment (start 131.400148 96.775851) (end 131.538132 96.567379) (width 0.1) (layer "F.Cu") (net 2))
 (segment (start 139.601022 102.503692) (end 139.739006 102.29522) (width 0.1) (layer "F.Cu") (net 2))
 (segment (start 139.187069 103.129106) (end 130.848211 97.609736) (width 0.1) (layer "F.Cu") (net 2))
 (segment (start 97.79294 98.792164) (end 98.04294 98.792164) (width 0.1) (layer "F.Cu") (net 2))
 (segment (start 138.497148 104.171464) (end 138.635132 103.962992) (width 0.1) (layer "F.Cu") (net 2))
 (segment (start 138.911101 103.546049) (end 130.572243 98.026679) (width 0.1) (layer "F.Cu") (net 2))
 (segment (start 100.29294 98.792164) (end 100.54294 98.792164) (width 0.1) (layer "F.Cu") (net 2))
 (segment (start 138.22118 104.588406) (end 138.359164 104.379935) (width 0.1) (layer "F.Cu") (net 2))
 (segment (start 100.04294 88.792164) (end 100.29294 88.792164) (width 0.1) (layer "F.Cu") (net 2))
 (segment (start 137.669243 105.422292) (end 137.807227 105.213821) (width 0.1) (layer "F.Cu") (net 2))
 (segment (start 101.29294 99.742164) (end 101.3 99.749224) (width 0.1) (layer "F.Cu") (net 2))
 (segment (start 138.635132 103.962992) (end 130.296274 98.443622) (width 0.1) (layer "F.Cu") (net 2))
 (segment (start 128.359611 99.2) (end 127.35 99.2) (width 0.1) (layer "F.Cu") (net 2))
 (segment (start 100.29294 88.792164) (end 100.29294 98.792164) (width 0.1) (layer "F.Cu") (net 2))
 (segment (start 137.807227 105.213821) (end 129.468369 99.694451) (width 0.1) (layer "F.Cu") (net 2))
 (segment (start 131.262164 96.984322) (end 139.601022 102.503692) (width 0.1) (layer "F.Cu") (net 2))
 (segment (start 96.54294 98.70706) (end 96.35 98.9) (width 0.1) (layer "F.Cu") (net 2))
 (segment (start 140.152959 101.669806) (end 140.290943 101.461335) (width 0.1) (layer "F.Cu") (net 2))
 (segment (start 131.12418 97.192793) (end 131.262164 96.984322) (width 0.1) (layer "F.Cu") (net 2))
 (segment (start 98.29294 98.792164) (end 98.54294 98.792164) (width 0.1) (layer "F.Cu") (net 2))
 (segment (start 100.54294 88.792164) (end 100.79294 88.792164) (width 0.1) (layer "F.Cu") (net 2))
 (segment (start 96.79294 88.792164) (end 96.79294 98.792164) (width 0.1) (layer "F.Cu") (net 2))
 (segment (start 139.739006 102.29522) (end 131.400148 96.775851) (width 0.1) (layer "F.Cu") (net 2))
 (segment (start 138.359164 104.379935) (end 130.020306 98.860565) (width 0.1) (layer "F.Cu") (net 2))
 (segment (start 99.79294 98.792164) (end 100.04294 98.792164) (width 0.1) (layer "F.Cu") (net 2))
 (segment (start 129.744337 99.277508) (end 129.882321 99.069037) (width 0.1) (layer "F.Cu") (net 2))
 (segment (start 97.29294 88.792164) (end 97.29294 98.792164) (width 0.1) (layer "F.Cu") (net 2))
 (segment (start 97.29294 98.792164) (end 97.54294 98.792164) (width 0.1) (layer "F.Cu") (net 2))
 (segment (start 100.54294 98.792164) (end 100.54294 88.792164) (width 0.1) (layer "F.Cu") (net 2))
 (segment (start 129.468369 99.694451) (end 129.606353 99.485979) (width 0.1) (layer "F.Cu") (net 2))
 (segment (start 97.54294 98.792164) (end 97.54294 88.792164) (width 0.1) (layer "F.Cu") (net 2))
 (via (at 102.95 102.25) (size 0.6) (drill 0.3) (layers "F.Cu" "B.Cu") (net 2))
 (via (at 124.4 99.2) (size 0.6) (drill 0.3) (layers "F.Cu" "B.Cu") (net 2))
 (segment (start 104.93 104.23) (end 104.93 105.3) (width 0.1) (layer "B.Cu") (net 2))
 (segment (start 106 99.2) (end 102.95 102.25) (width 0.1) (layer "B.Cu") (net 2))
 (segment (start 102.95 102.25) (end 104.93 104.23) (width 0.1) (layer "B.Cu") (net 2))
 (segment (start 124.4 99.2) (end 106 99.2) (width 0.1) (layer "B.Cu") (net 2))
 (segment (start 96.95 101.15) (end 98.842164 103.042164) (width 0.2) (layer "F.Cu") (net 3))
 (segment (start 96.4 100.6) (end 96.95 101.15) (width 0.2) (layer "F.Cu") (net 3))
 (segment (start 96.4 99.55) (end 96.35 99.5) (width 0.2) (layer "F.Cu") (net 3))
 (segment (start 110.292164 103.042164) (end 112.55 105.3) (width 0.2) (layer "F.Cu") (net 3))
 (segment (start 96.4 100.6) (end 96.4 99.55) (width 0.2) (layer "F.Cu") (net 3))
 (segment (start 98.842164 103.042164) (end 110.292164 103.042164) (width 0.2) (layer "F.Cu") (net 3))
 (segment (start 127.34 93.05) (end 129.6 93.05) (width 0.1) (layer "F.Cu") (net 6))
 (segment (start 130.8 93.2) (end 130.65 93.05) (width 0.1) (layer "F.Cu") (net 6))
 (segment (start 130.65 93.05) (end 129.6 93.05) (width 0.1) (layer "F.Cu") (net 6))
 (segment (start 131.1 93.2) (end 130.8 93.2) (width 0.1) (layer "F.Cu") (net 6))
 (segment (start 115.09 105.3) (end 127.34 93.05) (width 0.1) (layer "F.Cu") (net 6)))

